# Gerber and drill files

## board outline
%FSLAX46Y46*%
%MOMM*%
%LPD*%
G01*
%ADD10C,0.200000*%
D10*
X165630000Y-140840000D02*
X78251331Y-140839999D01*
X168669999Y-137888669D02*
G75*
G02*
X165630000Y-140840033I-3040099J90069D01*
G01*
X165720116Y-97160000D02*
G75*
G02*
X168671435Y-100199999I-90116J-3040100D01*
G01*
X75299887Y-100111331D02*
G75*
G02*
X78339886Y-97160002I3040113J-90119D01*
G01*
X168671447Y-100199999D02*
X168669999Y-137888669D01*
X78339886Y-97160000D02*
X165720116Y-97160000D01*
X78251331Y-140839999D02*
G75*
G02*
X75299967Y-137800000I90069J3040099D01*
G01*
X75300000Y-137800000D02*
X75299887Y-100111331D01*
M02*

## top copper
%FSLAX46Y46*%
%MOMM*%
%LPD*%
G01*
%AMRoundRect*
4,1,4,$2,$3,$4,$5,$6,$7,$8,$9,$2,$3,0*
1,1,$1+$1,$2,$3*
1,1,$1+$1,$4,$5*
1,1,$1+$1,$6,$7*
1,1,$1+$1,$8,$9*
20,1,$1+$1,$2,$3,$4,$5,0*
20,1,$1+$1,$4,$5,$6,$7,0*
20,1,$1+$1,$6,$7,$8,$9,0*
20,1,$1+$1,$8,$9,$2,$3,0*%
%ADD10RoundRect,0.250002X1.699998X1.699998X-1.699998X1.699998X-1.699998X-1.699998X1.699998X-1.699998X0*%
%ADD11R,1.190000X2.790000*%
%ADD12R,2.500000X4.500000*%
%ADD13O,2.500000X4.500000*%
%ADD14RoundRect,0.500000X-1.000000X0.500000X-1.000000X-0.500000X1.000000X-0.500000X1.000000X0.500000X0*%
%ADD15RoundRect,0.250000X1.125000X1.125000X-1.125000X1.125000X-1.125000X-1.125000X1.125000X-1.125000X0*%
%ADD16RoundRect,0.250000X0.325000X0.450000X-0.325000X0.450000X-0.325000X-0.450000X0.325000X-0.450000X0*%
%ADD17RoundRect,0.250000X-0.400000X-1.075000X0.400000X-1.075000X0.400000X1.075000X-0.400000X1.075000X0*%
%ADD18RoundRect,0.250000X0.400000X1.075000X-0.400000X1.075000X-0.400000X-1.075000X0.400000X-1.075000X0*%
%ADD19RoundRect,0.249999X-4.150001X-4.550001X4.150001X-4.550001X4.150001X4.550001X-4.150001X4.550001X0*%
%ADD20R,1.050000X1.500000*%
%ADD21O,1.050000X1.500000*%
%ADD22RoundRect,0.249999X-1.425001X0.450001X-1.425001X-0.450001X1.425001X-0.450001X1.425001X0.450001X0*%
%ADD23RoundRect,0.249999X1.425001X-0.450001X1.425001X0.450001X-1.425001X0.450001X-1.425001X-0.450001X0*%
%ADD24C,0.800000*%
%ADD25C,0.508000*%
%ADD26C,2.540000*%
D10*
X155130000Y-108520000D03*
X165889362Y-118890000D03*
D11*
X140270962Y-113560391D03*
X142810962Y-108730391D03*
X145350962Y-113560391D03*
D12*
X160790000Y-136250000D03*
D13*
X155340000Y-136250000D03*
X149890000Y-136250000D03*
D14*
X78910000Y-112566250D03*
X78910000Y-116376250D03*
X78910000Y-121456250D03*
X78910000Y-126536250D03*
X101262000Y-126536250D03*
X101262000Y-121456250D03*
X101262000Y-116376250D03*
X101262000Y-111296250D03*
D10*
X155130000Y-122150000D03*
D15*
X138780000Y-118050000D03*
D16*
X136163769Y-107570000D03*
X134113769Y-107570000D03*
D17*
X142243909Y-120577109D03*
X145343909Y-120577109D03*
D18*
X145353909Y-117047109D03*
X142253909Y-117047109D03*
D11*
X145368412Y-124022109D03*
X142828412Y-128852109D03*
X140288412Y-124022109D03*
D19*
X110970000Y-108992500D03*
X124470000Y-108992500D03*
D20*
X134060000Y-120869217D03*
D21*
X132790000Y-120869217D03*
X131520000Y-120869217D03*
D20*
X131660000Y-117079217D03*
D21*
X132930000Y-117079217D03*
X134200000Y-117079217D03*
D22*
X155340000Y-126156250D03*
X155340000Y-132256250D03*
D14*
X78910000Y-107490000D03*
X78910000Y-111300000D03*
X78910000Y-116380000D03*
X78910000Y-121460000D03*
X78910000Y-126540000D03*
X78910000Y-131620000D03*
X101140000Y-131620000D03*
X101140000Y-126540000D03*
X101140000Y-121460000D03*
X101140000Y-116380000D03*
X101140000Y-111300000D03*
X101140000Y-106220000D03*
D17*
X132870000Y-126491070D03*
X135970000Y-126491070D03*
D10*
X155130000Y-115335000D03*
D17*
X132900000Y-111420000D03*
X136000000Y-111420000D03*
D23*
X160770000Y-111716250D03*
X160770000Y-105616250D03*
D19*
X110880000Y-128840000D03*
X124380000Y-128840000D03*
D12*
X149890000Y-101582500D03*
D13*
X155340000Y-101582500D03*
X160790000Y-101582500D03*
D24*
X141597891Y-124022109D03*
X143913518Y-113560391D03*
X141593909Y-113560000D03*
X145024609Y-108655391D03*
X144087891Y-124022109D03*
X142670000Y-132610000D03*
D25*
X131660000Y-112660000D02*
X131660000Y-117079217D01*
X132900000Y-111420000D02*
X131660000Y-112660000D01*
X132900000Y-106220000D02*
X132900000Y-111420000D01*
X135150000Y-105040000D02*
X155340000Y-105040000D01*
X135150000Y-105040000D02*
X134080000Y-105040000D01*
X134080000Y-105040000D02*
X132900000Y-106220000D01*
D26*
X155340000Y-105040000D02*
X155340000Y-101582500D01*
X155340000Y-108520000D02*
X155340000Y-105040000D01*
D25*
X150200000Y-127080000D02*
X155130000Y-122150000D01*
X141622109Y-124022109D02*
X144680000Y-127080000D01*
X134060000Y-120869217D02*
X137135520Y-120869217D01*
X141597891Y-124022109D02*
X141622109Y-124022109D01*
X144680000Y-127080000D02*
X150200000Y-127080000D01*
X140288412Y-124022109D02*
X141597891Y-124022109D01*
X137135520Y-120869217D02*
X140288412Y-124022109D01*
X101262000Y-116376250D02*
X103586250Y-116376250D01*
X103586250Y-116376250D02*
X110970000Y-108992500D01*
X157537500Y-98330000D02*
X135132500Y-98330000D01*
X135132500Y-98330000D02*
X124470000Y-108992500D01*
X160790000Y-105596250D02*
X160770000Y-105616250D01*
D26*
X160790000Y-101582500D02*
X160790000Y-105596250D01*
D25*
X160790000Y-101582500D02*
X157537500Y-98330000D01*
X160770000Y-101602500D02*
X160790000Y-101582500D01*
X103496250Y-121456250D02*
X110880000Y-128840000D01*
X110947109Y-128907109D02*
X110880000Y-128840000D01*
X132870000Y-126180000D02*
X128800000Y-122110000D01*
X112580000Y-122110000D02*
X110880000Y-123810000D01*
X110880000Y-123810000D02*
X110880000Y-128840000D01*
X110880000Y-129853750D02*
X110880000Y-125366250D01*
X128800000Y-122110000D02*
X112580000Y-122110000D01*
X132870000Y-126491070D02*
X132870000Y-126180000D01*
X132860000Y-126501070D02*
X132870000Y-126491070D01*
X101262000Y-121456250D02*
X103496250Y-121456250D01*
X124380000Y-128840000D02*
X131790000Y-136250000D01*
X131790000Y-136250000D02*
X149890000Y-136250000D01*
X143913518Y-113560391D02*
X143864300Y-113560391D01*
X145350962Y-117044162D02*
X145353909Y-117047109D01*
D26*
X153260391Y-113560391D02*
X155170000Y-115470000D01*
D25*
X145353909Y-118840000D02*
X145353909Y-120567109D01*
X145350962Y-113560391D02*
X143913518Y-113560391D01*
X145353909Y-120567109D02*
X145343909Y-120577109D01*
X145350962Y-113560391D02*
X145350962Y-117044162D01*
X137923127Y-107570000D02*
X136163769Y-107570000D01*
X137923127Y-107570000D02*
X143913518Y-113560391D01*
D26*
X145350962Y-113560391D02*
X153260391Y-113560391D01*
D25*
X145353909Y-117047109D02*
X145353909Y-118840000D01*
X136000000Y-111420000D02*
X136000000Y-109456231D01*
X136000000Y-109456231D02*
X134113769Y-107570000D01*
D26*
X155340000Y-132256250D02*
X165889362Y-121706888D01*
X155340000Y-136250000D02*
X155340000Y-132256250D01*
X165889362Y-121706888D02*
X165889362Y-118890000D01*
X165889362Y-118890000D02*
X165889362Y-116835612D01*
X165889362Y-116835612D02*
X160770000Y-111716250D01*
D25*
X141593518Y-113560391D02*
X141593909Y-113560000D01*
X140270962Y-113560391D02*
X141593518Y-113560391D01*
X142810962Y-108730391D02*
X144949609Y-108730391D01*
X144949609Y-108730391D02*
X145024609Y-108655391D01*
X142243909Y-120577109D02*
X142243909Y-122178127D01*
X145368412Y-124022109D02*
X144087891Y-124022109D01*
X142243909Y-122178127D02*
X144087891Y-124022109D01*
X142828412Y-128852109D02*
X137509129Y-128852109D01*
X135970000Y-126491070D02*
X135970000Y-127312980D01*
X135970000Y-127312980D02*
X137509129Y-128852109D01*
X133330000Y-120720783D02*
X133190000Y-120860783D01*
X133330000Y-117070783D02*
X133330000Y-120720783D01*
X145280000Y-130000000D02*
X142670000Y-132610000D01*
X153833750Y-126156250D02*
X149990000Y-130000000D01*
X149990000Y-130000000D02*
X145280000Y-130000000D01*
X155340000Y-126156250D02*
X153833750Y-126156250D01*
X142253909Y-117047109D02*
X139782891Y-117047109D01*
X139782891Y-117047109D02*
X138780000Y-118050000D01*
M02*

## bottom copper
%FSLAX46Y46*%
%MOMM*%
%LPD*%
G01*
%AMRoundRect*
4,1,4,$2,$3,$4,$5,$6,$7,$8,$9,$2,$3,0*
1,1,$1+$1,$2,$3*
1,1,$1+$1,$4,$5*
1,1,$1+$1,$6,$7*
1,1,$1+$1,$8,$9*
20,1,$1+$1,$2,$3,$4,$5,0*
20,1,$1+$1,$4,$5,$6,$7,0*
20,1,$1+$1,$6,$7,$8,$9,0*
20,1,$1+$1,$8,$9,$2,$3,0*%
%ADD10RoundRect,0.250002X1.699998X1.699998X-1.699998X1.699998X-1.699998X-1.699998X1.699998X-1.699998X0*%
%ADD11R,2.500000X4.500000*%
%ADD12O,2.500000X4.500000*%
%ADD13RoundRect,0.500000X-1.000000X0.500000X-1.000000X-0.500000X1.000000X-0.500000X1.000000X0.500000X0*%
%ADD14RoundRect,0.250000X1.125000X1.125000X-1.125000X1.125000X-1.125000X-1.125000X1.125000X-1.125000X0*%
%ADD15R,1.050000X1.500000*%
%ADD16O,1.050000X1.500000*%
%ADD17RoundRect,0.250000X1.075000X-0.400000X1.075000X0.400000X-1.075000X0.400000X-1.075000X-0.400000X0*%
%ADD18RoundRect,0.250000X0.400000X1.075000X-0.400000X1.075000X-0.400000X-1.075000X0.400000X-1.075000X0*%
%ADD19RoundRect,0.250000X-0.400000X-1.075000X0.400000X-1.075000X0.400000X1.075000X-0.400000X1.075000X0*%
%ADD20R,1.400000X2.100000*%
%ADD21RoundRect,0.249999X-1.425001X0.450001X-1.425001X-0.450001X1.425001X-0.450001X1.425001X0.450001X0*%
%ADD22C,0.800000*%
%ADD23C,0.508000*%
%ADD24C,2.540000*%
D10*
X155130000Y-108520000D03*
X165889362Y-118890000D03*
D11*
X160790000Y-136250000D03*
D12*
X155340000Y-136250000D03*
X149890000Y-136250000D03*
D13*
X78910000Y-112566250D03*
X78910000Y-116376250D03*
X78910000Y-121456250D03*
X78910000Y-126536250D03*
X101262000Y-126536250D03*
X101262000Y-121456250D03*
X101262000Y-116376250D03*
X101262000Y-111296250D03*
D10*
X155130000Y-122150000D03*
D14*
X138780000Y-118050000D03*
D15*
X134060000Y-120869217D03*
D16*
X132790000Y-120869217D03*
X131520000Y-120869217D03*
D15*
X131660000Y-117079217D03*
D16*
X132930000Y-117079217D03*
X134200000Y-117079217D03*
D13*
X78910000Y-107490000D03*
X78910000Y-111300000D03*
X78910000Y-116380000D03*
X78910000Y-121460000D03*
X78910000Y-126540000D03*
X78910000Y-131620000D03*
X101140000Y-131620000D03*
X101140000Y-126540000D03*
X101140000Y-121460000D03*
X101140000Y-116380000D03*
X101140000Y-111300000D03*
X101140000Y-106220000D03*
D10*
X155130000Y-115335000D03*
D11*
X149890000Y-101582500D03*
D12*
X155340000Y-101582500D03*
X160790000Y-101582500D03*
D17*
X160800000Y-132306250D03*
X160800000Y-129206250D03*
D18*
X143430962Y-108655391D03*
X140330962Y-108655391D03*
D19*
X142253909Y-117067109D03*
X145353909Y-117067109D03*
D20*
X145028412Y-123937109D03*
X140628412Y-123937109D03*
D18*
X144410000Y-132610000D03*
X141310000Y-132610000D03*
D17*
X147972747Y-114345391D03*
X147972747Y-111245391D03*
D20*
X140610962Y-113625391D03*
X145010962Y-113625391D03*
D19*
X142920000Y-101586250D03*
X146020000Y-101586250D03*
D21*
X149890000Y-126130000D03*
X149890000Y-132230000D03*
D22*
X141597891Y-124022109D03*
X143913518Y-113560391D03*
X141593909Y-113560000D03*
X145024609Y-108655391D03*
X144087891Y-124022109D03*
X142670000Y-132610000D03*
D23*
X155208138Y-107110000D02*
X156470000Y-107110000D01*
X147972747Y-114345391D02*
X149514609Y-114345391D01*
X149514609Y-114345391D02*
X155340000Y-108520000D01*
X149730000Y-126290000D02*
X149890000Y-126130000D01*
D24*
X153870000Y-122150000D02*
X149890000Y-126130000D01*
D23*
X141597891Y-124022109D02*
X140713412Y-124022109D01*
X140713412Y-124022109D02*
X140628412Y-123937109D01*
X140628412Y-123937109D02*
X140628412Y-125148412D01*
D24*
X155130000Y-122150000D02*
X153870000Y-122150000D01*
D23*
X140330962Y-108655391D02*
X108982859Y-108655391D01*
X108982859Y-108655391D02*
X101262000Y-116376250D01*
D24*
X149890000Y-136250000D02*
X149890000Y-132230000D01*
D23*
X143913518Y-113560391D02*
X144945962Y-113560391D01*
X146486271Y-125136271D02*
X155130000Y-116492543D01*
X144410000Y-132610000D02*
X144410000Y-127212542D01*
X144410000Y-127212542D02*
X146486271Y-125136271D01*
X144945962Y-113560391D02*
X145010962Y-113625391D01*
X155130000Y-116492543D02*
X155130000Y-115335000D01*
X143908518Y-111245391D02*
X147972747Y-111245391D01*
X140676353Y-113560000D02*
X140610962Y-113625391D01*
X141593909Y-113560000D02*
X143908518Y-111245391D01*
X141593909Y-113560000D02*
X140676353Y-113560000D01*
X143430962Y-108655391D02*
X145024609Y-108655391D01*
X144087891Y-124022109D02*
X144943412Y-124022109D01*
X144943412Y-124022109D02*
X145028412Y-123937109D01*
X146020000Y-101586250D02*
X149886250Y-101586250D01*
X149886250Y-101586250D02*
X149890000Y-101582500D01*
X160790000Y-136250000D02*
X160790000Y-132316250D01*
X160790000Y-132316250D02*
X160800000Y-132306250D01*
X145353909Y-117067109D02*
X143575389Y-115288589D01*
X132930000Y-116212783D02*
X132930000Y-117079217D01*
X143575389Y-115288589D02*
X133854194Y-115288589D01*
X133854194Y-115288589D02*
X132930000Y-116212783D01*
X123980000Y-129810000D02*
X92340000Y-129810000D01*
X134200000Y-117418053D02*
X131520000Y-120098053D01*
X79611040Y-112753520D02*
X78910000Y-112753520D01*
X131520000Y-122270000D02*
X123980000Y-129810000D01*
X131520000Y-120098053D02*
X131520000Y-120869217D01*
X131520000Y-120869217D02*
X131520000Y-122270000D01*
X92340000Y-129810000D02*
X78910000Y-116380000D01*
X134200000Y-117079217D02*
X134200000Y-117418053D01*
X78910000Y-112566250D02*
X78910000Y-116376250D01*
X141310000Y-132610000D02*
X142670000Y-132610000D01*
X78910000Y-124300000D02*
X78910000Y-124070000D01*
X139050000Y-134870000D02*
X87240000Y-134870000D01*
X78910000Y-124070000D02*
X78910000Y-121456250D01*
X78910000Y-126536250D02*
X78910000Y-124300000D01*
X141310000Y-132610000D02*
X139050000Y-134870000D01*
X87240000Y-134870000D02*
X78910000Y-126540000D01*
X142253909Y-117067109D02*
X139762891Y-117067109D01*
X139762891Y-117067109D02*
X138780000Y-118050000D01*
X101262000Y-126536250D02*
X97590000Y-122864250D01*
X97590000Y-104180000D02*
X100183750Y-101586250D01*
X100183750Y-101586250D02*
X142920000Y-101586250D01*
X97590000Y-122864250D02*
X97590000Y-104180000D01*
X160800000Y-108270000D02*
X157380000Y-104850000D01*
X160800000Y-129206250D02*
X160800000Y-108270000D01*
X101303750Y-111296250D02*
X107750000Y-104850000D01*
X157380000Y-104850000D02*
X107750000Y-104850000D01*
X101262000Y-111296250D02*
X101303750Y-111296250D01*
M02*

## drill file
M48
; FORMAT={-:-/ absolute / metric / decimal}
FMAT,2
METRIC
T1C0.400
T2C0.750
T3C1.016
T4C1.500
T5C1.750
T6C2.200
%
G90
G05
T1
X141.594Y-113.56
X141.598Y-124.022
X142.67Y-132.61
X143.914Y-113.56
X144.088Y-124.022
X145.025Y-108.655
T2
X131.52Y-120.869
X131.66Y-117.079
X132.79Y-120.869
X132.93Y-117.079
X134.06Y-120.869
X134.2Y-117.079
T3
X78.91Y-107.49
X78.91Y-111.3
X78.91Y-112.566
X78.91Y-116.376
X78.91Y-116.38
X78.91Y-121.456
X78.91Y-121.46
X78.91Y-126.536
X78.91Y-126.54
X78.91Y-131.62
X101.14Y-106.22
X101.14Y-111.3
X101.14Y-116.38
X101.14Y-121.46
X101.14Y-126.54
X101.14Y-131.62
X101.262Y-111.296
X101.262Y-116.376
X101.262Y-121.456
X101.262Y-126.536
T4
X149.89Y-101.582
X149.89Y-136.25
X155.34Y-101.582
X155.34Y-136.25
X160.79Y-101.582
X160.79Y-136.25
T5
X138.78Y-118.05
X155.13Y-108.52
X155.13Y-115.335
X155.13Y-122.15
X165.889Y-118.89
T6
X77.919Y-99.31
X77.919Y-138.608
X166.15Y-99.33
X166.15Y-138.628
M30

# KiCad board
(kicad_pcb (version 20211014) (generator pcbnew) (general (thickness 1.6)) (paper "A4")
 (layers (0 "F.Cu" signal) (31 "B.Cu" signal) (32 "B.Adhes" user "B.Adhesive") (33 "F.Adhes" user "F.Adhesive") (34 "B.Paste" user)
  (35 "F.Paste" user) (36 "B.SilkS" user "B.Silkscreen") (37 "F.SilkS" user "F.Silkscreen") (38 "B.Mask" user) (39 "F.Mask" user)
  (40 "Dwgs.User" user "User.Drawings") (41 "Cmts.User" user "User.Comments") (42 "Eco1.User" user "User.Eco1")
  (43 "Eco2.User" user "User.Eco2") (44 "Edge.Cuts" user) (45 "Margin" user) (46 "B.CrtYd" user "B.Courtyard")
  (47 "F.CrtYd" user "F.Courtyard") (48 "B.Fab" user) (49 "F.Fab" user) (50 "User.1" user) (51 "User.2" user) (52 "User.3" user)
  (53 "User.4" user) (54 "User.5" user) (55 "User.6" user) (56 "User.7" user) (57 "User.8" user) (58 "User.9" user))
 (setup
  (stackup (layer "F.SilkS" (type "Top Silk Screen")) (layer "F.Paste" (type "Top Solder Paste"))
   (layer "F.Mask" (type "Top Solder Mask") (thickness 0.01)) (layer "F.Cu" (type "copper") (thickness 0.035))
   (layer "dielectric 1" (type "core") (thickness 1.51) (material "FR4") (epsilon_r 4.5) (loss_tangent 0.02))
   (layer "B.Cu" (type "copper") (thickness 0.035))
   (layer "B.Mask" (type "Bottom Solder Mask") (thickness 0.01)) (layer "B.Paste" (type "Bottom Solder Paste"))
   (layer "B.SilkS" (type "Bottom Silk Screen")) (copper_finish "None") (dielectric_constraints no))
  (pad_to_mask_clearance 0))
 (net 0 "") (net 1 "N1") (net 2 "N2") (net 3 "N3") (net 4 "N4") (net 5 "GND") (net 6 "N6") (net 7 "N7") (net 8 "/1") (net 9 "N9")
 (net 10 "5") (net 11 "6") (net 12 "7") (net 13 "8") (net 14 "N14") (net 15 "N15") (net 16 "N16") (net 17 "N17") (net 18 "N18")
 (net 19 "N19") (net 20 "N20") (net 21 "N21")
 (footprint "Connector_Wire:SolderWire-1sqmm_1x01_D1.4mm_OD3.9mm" (layer "F.Cu") (at 155.13 108.52 180)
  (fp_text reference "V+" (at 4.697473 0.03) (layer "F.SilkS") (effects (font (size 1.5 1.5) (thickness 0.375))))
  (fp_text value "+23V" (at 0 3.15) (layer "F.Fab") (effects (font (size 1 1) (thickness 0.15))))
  (pad "1" thru_hole roundrect locked (at 0 0 180) (size 3.9 3.9) (drill 1.75) (layers *.Cu *.Mask) (roundrect_rratio 0.064103) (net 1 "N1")))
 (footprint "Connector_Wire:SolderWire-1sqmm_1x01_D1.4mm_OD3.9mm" (layer "F.Cu") (at 165.889362 118.89 180)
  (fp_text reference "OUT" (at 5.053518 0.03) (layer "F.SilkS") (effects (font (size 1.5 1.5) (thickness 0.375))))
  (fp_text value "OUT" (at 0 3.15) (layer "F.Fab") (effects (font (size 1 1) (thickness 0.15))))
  (pad "1" thru_hole roundrect locked (at 0 0 180) (size 3.9 3.9) (drill 1.75) (layers *.Cu *.Mask) (roundrect_rratio 0.064103) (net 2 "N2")))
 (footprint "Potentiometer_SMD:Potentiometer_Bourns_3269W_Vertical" (layer "F.Cu") (at 142.810962 111.145391 180)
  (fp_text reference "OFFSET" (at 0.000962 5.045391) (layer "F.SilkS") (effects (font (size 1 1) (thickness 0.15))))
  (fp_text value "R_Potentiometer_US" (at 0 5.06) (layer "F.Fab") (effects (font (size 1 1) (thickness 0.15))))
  (pad "1" smd rect locked (at 2.54 -2.415 180) (size 1.19 2.79) (layers "F.Cu" "F.Paste" "F.Mask") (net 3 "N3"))
  (pad "2" smd rect locked (at 0 2.415 180) (size 1.19 2.79) (layers "F.Cu" "F.Paste" "F.Mask") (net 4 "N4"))
  (pad "3" smd rect locked (at -2.54 -2.415 180) (size 1.19 2.79) (layers "F.Cu" "F.Paste" "F.Mask") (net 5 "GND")))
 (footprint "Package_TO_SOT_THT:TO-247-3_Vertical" (layer "F.Cu") (at 160.79 136.25 180)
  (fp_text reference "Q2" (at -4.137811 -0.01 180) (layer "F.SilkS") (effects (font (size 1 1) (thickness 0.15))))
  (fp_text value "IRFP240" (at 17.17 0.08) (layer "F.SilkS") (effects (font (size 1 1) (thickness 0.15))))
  (pad "1" thru_hole rect locked (at 0 0 180) (size 2.5 4.5) (drill 1.5) (layers *.Cu *.Mask) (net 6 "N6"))
  (pad "2" thru_hole oval locked (at 5.45 0 180) (size 2.5 4.5) (drill 1.5) (layers *.Cu *.Mask) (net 2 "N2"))
  (pad "3" thru_hole oval locked (at 10.9 0 180) (size 2.5 4.5) (drill 1.5) (layers *.Cu *.Mask) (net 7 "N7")))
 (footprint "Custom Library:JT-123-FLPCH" (layer "F.Cu") (at 90.34 118.91625 -90)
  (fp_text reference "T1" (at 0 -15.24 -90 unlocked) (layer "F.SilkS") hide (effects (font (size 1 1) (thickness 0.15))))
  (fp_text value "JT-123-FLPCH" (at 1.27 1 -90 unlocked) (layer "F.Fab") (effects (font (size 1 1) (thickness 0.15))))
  (pad "1" thru_hole roundrect locked (at -6.35 11.43 270) (size 2 3) (drill 1.016) (layers *.Cu *.Mask) (roundrect_rratio 0.25)
   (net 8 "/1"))
  (pad "2" thru_hole roundrect locked (at -2.54 11.43 270) (size 2 3) (drill 1.016) (layers *.Cu *.Mask) (roundrect_rratio 0.25)
   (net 8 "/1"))
  (pad "3" thru_hole roundrect locked (at 2.54 11.43 270) (size 2 3) (drill 1.016) (layers *.Cu *.Mask) (roundrect_rratio 0.25) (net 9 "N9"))
  (pad "4" thru_hole roundrect locked (at 7.62 11.43 270) (size 2 3) (drill 1.016) (layers *.Cu *.Mask) (roundrect_rratio 0.25) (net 9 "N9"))
  (pad "5" thru_hole roundrect locked (at 7.62 -10.922 270) (size 2 3) (drill 1.016) (layers *.Cu *.Mask) (roundrect_rratio 0.25)
   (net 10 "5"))
  (pad "6" thru_hole roundrect locked (at 2.54 -10.922 270) (size 2 3) (drill 1.016) (layers *.Cu *.Mask) (roundrect_rratio 0.25)
   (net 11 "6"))
  (pad "7" thru_hole roundrect locked (at -2.54 -10.922 270) (size 2 3) (drill 1.016) (layers *.Cu *.Mask) (roundrect_rratio 0.25)
   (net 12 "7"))
  (pad "8" thru_hole roundrect locked (at -7.62 -10.922 270) (size 2 3) (drill 1.016) (layers *.Cu *.Mask) (roundrect_rratio 0.25)
   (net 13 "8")))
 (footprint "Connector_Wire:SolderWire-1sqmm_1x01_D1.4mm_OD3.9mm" (layer "F.Cu") (at 155.13 122.15 180)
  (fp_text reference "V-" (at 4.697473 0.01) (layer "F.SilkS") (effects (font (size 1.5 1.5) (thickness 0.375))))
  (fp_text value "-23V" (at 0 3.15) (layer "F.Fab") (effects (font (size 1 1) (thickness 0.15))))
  (pad "1" thru_hole roundrect locked (at 0 0 180) (size 3.9 3.9) (drill 1.75) (layers *.Cu *.Mask) (roundrect_rratio 0.064103)
   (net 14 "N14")))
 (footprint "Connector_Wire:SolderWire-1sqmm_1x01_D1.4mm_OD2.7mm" (layer "F.Cu") (at 138.78 118.05 180)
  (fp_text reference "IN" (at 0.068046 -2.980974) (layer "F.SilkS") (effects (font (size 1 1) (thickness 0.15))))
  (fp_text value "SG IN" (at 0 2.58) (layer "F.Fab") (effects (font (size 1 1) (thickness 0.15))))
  (pad "1" thru_hole roundrect locked (at 0 0 180) (size 2.75 2.75) (drill 1.75) (layers *.Cu *.Mask) (roundrect_rratio 0.090909)
   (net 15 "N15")))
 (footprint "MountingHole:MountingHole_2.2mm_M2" (layer "F.Cu") (at 166.15 138.627795)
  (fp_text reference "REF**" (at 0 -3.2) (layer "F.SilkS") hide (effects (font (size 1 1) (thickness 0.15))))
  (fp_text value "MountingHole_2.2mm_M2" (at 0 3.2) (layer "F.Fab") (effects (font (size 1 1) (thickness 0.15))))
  (pad "" np_thru_hole circle locked (at 0 0) (size 2.2 2.2) (drill 2.2) (layers *.Cu *.Mask)))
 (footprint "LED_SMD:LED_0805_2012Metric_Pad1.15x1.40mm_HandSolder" (layer "F.Cu") (at 135.138769 107.57 180)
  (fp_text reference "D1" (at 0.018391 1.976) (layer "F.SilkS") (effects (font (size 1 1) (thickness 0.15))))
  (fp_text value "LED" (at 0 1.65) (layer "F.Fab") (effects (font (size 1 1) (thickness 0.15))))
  (pad "1" smd roundrect locked (at -1.025 0 180) (size 1.15 1.4) (layers "F.Cu" "F.Paste" "F.Mask") (roundrect_rratio 0.217391)
   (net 5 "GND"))
  (pad "2" smd roundrect locked (at 1.025 0 180) (size 1.15 1.4) (layers "F.Cu" "F.Paste" "F.Mask") (roundrect_rratio 0.217391)
   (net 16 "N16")))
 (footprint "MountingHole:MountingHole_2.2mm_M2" (layer "F.Cu") (at 77.918758 99.31)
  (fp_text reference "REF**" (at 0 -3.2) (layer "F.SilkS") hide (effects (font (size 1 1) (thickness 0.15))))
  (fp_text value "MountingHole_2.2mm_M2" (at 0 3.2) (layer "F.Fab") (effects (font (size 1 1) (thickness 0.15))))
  (pad "" np_thru_hole circle locked (at 0 0) (size 2.2 2.2) (drill 2.2) (layers *.Cu *.Mask)))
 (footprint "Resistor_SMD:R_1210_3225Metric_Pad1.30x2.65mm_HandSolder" (layer "F.Cu") (at 143.793909 120.577109)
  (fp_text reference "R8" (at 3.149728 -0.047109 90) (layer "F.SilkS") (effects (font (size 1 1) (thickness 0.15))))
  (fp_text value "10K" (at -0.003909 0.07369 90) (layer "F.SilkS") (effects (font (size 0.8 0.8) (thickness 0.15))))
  (pad "1" smd roundrect locked (at -1.55 0) (size 1.3 2.65) (layers "F.Cu" "F.Paste" "F.Mask") (roundrect_rratio 0.192308) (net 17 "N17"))
  (pad "2" smd roundrect locked (at 1.55 0) (size 1.3 2.65) (layers "F.Cu" "F.Paste" "F.Mask") (roundrect_rratio 0.192308) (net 5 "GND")))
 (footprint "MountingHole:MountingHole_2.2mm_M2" (layer "F.Cu") (at 166.15 99.33)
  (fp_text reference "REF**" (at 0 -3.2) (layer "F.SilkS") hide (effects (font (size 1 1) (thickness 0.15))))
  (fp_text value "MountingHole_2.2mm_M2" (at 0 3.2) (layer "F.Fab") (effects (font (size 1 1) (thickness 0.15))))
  (pad "" np_thru_hole circle locked (at 0 0) (size 2.2 2.2) (drill 2.2) (layers *.Cu *.Mask)))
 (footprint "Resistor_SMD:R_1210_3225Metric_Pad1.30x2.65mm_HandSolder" (layer "F.Cu") (at 143.803909 117.047109 180)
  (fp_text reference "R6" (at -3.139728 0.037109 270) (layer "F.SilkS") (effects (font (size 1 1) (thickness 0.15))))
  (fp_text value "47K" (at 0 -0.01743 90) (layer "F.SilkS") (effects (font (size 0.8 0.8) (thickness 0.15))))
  (pad "1" smd roundrect locked (at -1.55 0 180) (size 1.3 2.65) (layers "F.Cu" "F.Paste" "F.Mask") (roundrect_rratio 0.192308)
   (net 5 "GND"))
  (pad "2" smd roundrect locked (at 1.55 0 180) (size 1.3 2.65) (layers "F.Cu" "F.Paste" "F.Mask") (roundrect_rratio 0.192308)
   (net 15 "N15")))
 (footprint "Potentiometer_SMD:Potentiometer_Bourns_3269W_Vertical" (layer "F.Cu") (at 142.828412 126.437109)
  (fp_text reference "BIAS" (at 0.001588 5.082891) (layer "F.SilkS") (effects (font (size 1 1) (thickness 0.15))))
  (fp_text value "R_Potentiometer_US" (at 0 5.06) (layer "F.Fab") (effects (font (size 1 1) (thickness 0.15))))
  (pad "1" smd rect locked (at 2.54 -2.415) (size 1.19 2.79) (layers "F.Cu" "F.Paste" "F.Mask") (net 17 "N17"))
  (pad "2" smd rect locked (at 0 2.415) (size 1.19 2.79) (layers "F.Cu" "F.Paste" "F.Mask") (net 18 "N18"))
  (pad "3" smd rect locked (at -2.54 -2.415) (size 1.19 2.79) (layers "F.Cu" "F.Paste" "F.Mask") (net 14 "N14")))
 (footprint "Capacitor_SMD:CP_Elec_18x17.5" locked (layer "F.Cu") (at 117.72 108.9925)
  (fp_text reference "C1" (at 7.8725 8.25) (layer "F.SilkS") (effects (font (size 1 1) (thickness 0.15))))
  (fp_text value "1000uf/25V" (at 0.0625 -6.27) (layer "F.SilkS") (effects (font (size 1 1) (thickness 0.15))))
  (pad "1" smd roundrect locked (at -6.75 0) (size 8.8 9.6) (layers "F.Cu" "F.Paste" "F.Mask") (roundrect_rratio 0.028409) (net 12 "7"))
  (pad "2" smd roundrect locked (at 6.75 0) (size 8.8 9.6) (layers "F.Cu" "F.Paste" "F.Mask") (roundrect_rratio 0.028409) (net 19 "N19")))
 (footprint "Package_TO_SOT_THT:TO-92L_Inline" (layer "F.Cu") (at 134.06 120.869217 180)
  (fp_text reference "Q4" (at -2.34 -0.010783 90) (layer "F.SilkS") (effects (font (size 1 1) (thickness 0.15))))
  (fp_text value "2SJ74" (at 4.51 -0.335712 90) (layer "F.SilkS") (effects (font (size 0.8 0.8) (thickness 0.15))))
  (pad "1" thru_hole rect locked (at 0 0 180) (size 1.05 1.5) (drill 0.75) (layers *.Cu *.Mask) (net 14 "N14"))
  (pad "2" thru_hole oval locked (at 1.27 0 180) (size 1.05 1.5) (drill 0.75) (layers *.Cu *.Mask) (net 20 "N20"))
  (pad "3" thru_hole oval locked (at 2.54 0 180) (size 1.05 1.5) (drill 0.75) (layers *.Cu *.Mask) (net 8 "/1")))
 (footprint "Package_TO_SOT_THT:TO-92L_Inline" (layer "F.Cu") (at 131.66 117.079217)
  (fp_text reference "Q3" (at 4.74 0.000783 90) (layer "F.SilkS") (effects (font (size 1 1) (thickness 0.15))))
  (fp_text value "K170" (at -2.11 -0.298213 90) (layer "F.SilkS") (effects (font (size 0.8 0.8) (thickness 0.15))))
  (pad "1" thru_hole rect locked (at 0 0) (size 1.05 1.5) (drill 0.75) (layers *.Cu *.Mask) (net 1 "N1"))
  (pad "2" thru_hole oval locked (at 1.27 0) (size 1.05 1.5) (drill 0.75) (layers *.Cu *.Mask) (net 20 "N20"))
  (pad "3" thru_hole oval locked (at 2.54 0) (size 1.05 1.5) (drill 0.75) (layers *.Cu *.Mask) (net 8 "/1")))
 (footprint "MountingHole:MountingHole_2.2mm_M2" (layer "F.Cu") (at 77.918758 138.607795)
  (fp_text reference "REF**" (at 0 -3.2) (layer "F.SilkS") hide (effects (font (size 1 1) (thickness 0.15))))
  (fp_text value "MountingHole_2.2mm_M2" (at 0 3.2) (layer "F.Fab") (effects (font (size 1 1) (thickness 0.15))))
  (pad "" np_thru_hole circle locked (at 0 0) (size 2.2 2.2) (drill 2.2) (layers *.Cu *.Mask)))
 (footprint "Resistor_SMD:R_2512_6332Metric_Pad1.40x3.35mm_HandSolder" (layer "F.Cu") (at 155.34 129.20625 -90)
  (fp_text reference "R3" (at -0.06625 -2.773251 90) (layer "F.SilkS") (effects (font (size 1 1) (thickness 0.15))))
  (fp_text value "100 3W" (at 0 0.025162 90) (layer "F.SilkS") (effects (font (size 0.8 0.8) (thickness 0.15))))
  (pad "1" smd roundrect locked (at -3.05 0 270) (size 1.4 3.35) (layers "F.Cu" "F.Paste" "F.Mask") (roundrect_rratio 0.178571) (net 9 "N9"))
  (pad "2" smd roundrect locked (at 3.05 0 270) (size 1.4 3.35) (layers "F.Cu" "F.Paste" "F.Mask") (roundrect_rratio 0.178571) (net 2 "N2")))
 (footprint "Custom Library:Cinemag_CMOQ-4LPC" (layer "F.Cu") (at 90.025 118.92 -90)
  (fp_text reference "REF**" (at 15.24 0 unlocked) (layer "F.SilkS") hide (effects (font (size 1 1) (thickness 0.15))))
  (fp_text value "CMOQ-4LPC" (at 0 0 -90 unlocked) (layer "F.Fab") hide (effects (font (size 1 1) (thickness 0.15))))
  (pad "1" thru_hole roundrect (at -11.43 11.115 270) (size 2 3) (drill 1.016) (layers *.Cu *.Mask) (roundrect_rratio 0.25))
  (pad "2" thru_hole roundrect (at -7.62 11.115 270) (size 2 3) (drill 1.016) (layers *.Cu *.Mask) (roundrect_rratio 0.25) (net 8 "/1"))
  (pad "3" thru_hole roundrect (at -2.54 11.115 270) (size 2 3) (drill 1.016) (layers *.Cu *.Mask) (roundrect_rratio 0.25) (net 8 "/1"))
  (pad "4" thru_hole roundrect (at 2.54 11.115 270) (size 2 3) (drill 1.016) (layers *.Cu *.Mask) (roundrect_rratio 0.25) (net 9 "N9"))
  (pad "5" thru_hole roundrect (at 7.62 11.115 270) (size 2 3) (drill 1.016) (layers *.Cu *.Mask) (roundrect_rratio 0.25) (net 9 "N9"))
  (pad "6" thru_hole roundrect (at 12.7 11.115 270) (size 2 3) (drill 1.016) (layers *.Cu *.Mask) (roundrect_rratio 0.25))
  (pad "7" thru_hole roundrect (at 12.7 -11.115 270) (size 2 3) (drill 1.016) (layers *.Cu *.Mask) (roundrect_rratio 0.25))
  (pad "8" thru_hole roundrect (at 7.62 -11.115 270) (size 2 3) (drill 1.016) (layers *.Cu *.Mask) (roundrect_rratio 0.25))
  (pad "9" thru_hole roundrect (at 2.54 -11.115 270) (size 2 3) (drill 1.016) (layers *.Cu *.Mask) (roundrect_rratio 0.25))
  (pad "10" thru_hole roundrect (at -2.54 -11.115 270) (size 2 3) (drill 1.016) (layers *.Cu *.Mask) (roundrect_rratio 0.25))
  (pad "11" thru_hole roundrect (at -7.62 -11.115 270) (size 2 3) (drill 1.016) (layers *.Cu *.Mask) (roundrect_rratio 0.25) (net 13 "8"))
  (pad "12" thru_hole roundrect (at -12.7 -11.115 270) (size 2 3) (drill 1.016) (layers *.Cu *.Mask) (roundrect_rratio 0.25)))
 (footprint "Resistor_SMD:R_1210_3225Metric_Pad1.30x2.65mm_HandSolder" (layer "F.Cu") (at 134.42 126.49107)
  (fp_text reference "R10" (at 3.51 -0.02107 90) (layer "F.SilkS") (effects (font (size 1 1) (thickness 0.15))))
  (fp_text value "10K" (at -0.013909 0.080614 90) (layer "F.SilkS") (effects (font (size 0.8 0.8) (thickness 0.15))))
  (pad "1" smd roundrect locked (at -1.55 0) (size 1.3 2.65) (layers "F.Cu" "F.Paste" "F.Mask") (roundrect_rratio 0.192308) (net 11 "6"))
  (pad "2" smd roundrect locked (at 1.55 0) (size 1.3 2.65) (layers "F.Cu" "F.Paste" "F.Mask") (roundrect_rratio 0.192308) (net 18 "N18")))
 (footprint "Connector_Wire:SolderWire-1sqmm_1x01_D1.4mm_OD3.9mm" (layer "F.Cu") (at 155.13 115.335 180)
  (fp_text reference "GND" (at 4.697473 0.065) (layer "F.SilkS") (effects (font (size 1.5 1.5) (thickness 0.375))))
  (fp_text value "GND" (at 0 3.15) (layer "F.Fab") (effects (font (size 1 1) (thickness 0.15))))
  (pad "1" thru_hole roundrect locked (at 0 0 180) (size 3.9 3.9) (drill 1.75) (layers *.Cu *.Mask) (roundrect_rratio 0.064103)
   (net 5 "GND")))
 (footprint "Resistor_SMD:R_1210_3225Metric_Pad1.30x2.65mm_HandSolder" (layer "F.Cu") (at 134.45 111.42)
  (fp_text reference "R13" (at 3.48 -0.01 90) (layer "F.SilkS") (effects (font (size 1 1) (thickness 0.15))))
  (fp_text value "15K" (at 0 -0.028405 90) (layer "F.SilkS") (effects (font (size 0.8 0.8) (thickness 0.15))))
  (pad "1" smd roundrect locked (at -1.55 0) (size 1.3 2.65) (layers "F.Cu" "F.Paste" "F.Mask") (roundrect_rratio 0.192308) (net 1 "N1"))
  (pad "2" smd roundrect locked (at 1.55 0) (size 1.3 2.65) (layers "F.Cu" "F.Paste" "F.Mask") (roundrect_rratio 0.192308) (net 16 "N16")))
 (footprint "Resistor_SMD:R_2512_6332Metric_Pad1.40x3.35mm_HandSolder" (layer "F.Cu") (at 160.77 108.66625 90)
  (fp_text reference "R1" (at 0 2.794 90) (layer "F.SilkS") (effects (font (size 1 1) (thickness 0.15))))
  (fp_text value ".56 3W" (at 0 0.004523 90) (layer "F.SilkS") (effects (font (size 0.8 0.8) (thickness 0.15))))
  (pad "1" smd roundrect locked (at -3.05 0 90) (size 1.4 3.35) (layers "F.Cu" "F.Paste" "F.Mask") (roundrect_rratio 0.178571) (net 2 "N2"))
  (pad "2" smd roundrect locked (at 3.05 0 90) (size 1.4 3.35) (layers "F.Cu" "F.Paste" "F.Mask") (roundrect_rratio 0.178571) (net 19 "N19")))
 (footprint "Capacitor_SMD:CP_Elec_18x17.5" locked (layer "F.Cu") (at 117.63 128.84)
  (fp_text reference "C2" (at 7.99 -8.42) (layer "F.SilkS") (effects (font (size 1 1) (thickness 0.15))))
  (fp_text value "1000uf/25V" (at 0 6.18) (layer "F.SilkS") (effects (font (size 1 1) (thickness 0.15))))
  (pad "1" smd roundrect locked (at -6.75 0) (size 8.8 9.6) (layers "F.Cu" "F.Paste" "F.Mask") (roundrect_rratio 0.028409) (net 11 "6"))
  (pad "2" smd roundrect locked (at 6.75 0) (size 8.8 9.6) (layers "F.Cu" "F.Paste" "F.Mask") (roundrect_rratio 0.028409) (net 7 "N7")))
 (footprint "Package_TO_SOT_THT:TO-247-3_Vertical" (layer "F.Cu") (at 149.89 101.5825)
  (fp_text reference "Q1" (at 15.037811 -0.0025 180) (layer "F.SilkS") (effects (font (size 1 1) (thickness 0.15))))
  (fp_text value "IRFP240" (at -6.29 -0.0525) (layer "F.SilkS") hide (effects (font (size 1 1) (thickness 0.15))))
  (pad "1" thru_hole rect locked (at 0 0) (size 2.5 4.5) (drill 1.5) (layers *.Cu *.Mask) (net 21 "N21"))
  (pad "2" thru_hole oval locked (at 5.45 0) (size 2.5 4.5) (drill 1.5) (layers *.Cu *.Mask) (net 1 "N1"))
  (pad "3" thru_hole oval locked (at 10.9 0) (size 2.5 4.5) (drill 1.5) (layers *.Cu *.Mask) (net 19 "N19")))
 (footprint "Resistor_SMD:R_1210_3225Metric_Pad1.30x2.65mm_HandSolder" (layer "B.Cu") (at 160.8 130.75625 90)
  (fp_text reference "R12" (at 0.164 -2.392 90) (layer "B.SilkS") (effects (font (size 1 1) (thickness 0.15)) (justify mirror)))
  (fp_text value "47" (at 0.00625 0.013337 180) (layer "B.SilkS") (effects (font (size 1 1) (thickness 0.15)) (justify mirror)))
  (pad "1" smd roundrect locked (at -1.55 0 90) (size 1.3 2.65) (layers "B.Cu" "B.Paste" "B.Mask") (roundrect_rratio 0.192308) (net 6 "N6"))
  (pad "2" smd roundrect locked (at 1.55 0 90) (size 1.3 2.65) (layers "B.Cu" "B.Paste" "B.Mask") (roundrect_rratio 0.192308) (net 13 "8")))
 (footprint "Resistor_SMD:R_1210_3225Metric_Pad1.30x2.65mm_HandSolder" (layer "B.Cu") (at 141.880962 108.655391 180)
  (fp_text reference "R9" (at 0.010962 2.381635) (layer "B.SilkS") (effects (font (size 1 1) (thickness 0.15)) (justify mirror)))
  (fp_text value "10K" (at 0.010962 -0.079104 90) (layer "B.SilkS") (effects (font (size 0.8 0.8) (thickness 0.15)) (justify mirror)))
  (pad "1" smd roundrect locked (at -1.55 0 180) (size 1.3 2.65) (layers "B.Cu" "B.Paste" "B.Mask") (roundrect_rratio 0.192308) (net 4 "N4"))
  (pad "2" smd roundrect locked (at 1.55 0 180) (size 1.3 2.65) (layers "B.Cu" "B.Paste" "B.Mask") (roundrect_rratio 0.192308) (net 12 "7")))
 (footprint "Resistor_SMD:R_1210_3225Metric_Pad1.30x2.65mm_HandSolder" (layer "B.Cu") (at 143.803909 117.067109)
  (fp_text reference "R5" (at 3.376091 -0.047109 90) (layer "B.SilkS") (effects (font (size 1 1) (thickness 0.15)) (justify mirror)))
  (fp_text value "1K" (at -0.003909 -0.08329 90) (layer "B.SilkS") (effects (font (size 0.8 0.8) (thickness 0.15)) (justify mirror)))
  (pad "1" smd roundrect locked (at -1.55 0) (size 1.3 2.65) (layers "B.Cu" "B.Paste" "B.Mask") (roundrect_rratio 0.192308) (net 15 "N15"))
  (pad "2" smd roundrect locked (at 1.55 0) (size 1.3 2.65) (layers "B.Cu" "B.Paste" "B.Mask") (roundrect_rratio 0.192308) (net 20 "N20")))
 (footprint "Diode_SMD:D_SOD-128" (layer "B.Cu") (at 142.828412 123.937109 180)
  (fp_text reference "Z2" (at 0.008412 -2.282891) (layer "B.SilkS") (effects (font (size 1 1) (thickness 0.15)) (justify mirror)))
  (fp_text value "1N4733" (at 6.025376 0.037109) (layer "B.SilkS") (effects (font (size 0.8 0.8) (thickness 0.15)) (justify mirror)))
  (pad "1" smd rect locked (at -2.2 0 180) (size 1.4 2.1) (layers "B.Cu" "B.Paste" "B.Mask") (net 17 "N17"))
  (pad "2" smd rect locked (at 2.2 0 180) (size 1.4 2.1) (layers "B.Cu" "B.Paste" "B.Mask") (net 14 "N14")))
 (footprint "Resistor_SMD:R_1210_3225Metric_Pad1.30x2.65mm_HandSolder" (layer "B.Cu") (at 142.86 132.61 180)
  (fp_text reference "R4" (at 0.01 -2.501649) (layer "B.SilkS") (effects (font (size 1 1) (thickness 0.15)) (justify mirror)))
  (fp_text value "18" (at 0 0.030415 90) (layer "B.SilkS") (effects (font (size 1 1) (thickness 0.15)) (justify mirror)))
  (pad "1" smd roundrect locked (at -1.55 0 180) (size 1.3 2.65) (layers "B.Cu" "B.Paste" "B.Mask") (roundrect_rratio 0.192308)
   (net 5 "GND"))
  (pad "2" smd roundrect locked (at 1.55 0 180) (size 1.3 2.65) (layers "B.Cu" "B.Paste" "B.Mask") (roundrect_rratio 0.192308) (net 9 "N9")))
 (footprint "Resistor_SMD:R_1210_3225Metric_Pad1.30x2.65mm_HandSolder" (layer "B.Cu") (at 147.972747 112.795391 90)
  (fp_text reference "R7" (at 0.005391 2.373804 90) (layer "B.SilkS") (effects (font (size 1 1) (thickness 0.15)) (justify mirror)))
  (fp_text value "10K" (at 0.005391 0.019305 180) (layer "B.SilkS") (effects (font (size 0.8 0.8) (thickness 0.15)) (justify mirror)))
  (pad "1" smd roundrect locked (at -1.55 0 90) (size 1.3 2.65) (layers "B.Cu" "B.Paste" "B.Mask") (roundrect_rratio 0.192308) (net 1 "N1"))
  (pad "2" smd roundrect locked (at 1.55 0 90) (size 1.3 2.65) (layers "B.Cu" "B.Paste" "B.Mask") (roundrect_rratio 0.192308) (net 3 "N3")))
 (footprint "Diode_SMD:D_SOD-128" (layer "B.Cu") (at 142.810962 113.625391)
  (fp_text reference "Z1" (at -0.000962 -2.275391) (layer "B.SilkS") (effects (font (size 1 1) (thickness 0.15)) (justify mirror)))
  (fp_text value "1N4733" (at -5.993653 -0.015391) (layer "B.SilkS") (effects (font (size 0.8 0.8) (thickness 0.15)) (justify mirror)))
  (pad "1" smd rect locked (at -2.2 0) (size 1.4 2.1) (layers "B.Cu" "B.Paste" "B.Mask") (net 3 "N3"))
  (pad "2" smd rect locked (at 2.2 0) (size 1.4 2.1) (layers "B.Cu" "B.Paste" "B.Mask") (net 5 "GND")))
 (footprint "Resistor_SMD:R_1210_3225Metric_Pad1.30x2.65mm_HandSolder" (layer "B.Cu") (at 144.47 101.58625)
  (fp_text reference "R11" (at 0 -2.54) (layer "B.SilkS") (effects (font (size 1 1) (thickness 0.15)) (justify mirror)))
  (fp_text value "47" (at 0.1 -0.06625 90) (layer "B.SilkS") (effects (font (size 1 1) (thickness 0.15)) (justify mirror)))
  (pad "1" smd roundrect locked (at -1.55 0) (size 1.3 2.65) (layers "B.Cu" "B.Paste" "B.Mask") (roundrect_rratio 0.192308) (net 10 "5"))
  (pad "2" smd roundrect locked (at 1.55 0) (size 1.3 2.65) (layers "B.Cu" "B.Paste" "B.Mask") (roundrect_rratio 0.192308) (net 21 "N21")))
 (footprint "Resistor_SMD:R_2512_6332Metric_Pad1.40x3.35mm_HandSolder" (layer "B.Cu") (at 149.89 129.18 -90)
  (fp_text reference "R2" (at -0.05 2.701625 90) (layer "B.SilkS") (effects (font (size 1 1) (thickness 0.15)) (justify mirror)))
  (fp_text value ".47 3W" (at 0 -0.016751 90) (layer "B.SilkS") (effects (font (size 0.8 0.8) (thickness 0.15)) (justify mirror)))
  (pad "1" smd roundrect locked (at -3.05 0 270) (size 1.4 3.35) (layers "B.Cu" "B.Paste" "B.Mask") (roundrect_rratio 0.178571)
   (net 14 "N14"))
  (pad "2" smd roundrect locked (at 3.05 0 270) (size 1.4 3.35) (layers "B.Cu" "B.Paste" "B.Mask") (roundrect_rratio 0.178571) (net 7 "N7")))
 (gr_line (start 165.63 140.84) (end 78.251331 140.839999) (layer "Edge.Cuts") (width 0.2))
 (gr_arc (start 168.669999 137.888669) (mid 167.748455 139.980769) (end 165.63 140.84) (layer "Edge.Cuts") (width 0.2))
 (gr_arc (start 165.720116 97.16) (mid 167.812216 98.081544) (end 168.671447 100.199999) (layer "Edge.Cuts") (width 0.2))
 (gr_arc (start 75.299887 100.111331) (mid 76.221431 98.019231) (end 78.339886 97.16) (layer "Edge.Cuts") (width 0.2))
 (gr_line (start 168.671447 100.199999) (end 168.669999 137.888669) (layer "Edge.Cuts") (width 0.2))
 (gr_line (start 78.339886 97.16) (end 165.720116 97.16) (layer "Edge.Cuts") (width 0.2))
 (gr_arc (start 78.251331 140.839999) (mid 76.159231 139.918455) (end 75.3 137.8) (layer "Edge.Cuts") (width 0.2))
 (gr_line (start 75.3 137.8) (end 75.299887 100.111331) (layer "Edge.Cuts") (width 0.2))
 (segment (start 131.66 112.66) (end 131.66 117.079217) (width 0.508) (layer "F.Cu") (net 1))
 (segment (start 132.9 111.42) (end 131.66 112.66) (width 0.508) (layer "F.Cu") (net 1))
 (segment (start 132.9 106.22) (end 132.9 111.42) (width 0.508) (layer "F.Cu") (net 1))
 (segment (start 135.15 105.04) (end 155.34 105.04) (width 0.508) (layer "F.Cu") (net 1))
 (segment (start 135.15 105.04) (end 134.08 105.04) (width 0.508) (layer "F.Cu") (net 1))
 (segment (start 134.08 105.04) (end 132.9 106.22) (width 0.508) (layer "F.Cu") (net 1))
 (segment (start 155.34 105.04) (end 155.34 101.5825) (width 2.54) (layer "F.Cu") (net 1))
 (segment (start 155.34 108.52) (end 155.34 105.04) (width 2.54) (layer "F.Cu") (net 1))
 (segment (start 155.208138 107.11) (end 156.47 107.11) (width 0.508) (layer "B.Cu") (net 1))
 (segment (start 147.972747 114.345391) (end 149.514609 114.345391) (width 0.508) (layer "B.Cu") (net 1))
 (segment (start 149.514609 114.345391) (end 155.34 108.52) (width 0.508) (layer "B.Cu") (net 1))
 (segment (start 150.2 127.08) (end 155.13 122.15) (width 0.508) (layer "F.Cu") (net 14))
 (segment (start 141.622109 124.022109) (end 144.68 127.08) (width 0.508) (layer "F.Cu") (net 14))
 (segment (start 134.06 120.869217) (end 137.13552 120.869217) (width 0.508) (layer "F.Cu") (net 14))
 (segment (start 141.597891 124.022109) (end 141.622109 124.022109) (width 0.508) (layer "F.Cu") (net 14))
 (segment (start 144.68 127.08) (end 150.2 127.08) (width 0.508) (layer "F.Cu") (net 14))
 (segment (start 140.288412 124.022109) (end 141.597891 124.022109) (width 0.508) (layer "F.Cu") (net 14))
 (segment (start 137.13552 120.869217) (end 140.288412 124.022109) (width 0.508) (layer "F.Cu") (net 14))
 (via (at 141.597891 124.022109) (size 0.8) (drill 0.4) (layers "F.Cu" "B.Cu") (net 14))
 (segment (start 149.73 126.29) (end 149.89 126.13) (width 0.508) (layer "B.Cu") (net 14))
 (segment (start 153.87 122.15) (end 149.89 126.13) (width 2.54) (layer "B.Cu") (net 14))
 (segment (start 141.597891 124.022109) (end 140.713412 124.022109) (width 0.508) (layer "B.Cu") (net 14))
 (segment (start 140.713412 124.022109) (end 140.628412 123.937109) (width 0.508) (layer "B.Cu") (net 14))
 (segment (start 140.628412 123.937109) (end 140.628412 125.148412) (width 0.508) (layer "B.Cu") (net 14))
 (segment (start 155.13 122.15) (end 153.87 122.15) (width 2.54) (layer "B.Cu") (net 14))
 (segment (start 101.262 116.37625) (end 103.58625 116.37625) (width 0.508) (layer "F.Cu") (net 12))
 (segment (start 103.58625 116.37625) (end 110.97 108.9925) (width 0.508) (layer "F.Cu") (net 12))
 (segment (start 140.330962 108.655391) (end 108.982859 108.655391) (width 0.508) (layer "B.Cu") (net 12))
 (segment (start 108.982859 108.655391) (end 101.262 116.37625) (width 0.508) (layer "B.Cu") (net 12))
 (segment (start 157.5375 98.33) (end 135.1325 98.33) (width 0.508) (layer "F.Cu") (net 19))
 (segment (start 135.1325 98.33) (end 124.47 108.9925) (width 0.508) (layer "F.Cu") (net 19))
 (segment (start 160.79 105.59625) (end 160.77 105.61625) (width 0.508) (layer "F.Cu") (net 19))
 (segment (start 160.79 101.5825) (end 160.79 105.59625) (width 2.54) (layer "F.Cu") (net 19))
 (segment (start 160.79 101.5825) (end 157.5375 98.33) (width 0.508) (layer "F.Cu") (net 19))
 (segment (start 160.77 101.6025) (end 160.79 101.5825) (width 0.508) (layer "F.Cu") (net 19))
 (segment (start 103.49625 121.45625) (end 110.88 128.84) (width 0.508) (layer "F.Cu") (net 11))
 (segment (start 110.947109 128.907109) (end 110.88 128.84) (width 0.508) (layer "F.Cu") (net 11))
 (segment (start 132.87 126.18) (end 128.8 122.11) (width 0.508) (layer "F.Cu") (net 11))
 (segment (start 112.58 122.11) (end 110.88 123.81) (width 0.508) (layer "F.Cu") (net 11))
 (segment (start 110.88 123.81) (end 110.88 128.84) (width 0.508) (layer "F.Cu") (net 11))
 (segment (start 110.88 129.85375) (end 110.88 125.36625) (width 0.508) (layer "F.Cu") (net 11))
 (segment (start 128.8 122.11) (end 112.58 122.11) (width 0.508) (layer "F.Cu") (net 11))
 (segment (start 132.87 126.49107) (end 132.87 126.18) (width 0.508) (layer "F.Cu") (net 11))
 (segment (start 132.86 126.50107) (end 132.87 126.49107) (width 0.508) (layer "F.Cu") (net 11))
 (segment (start 101.262 121.45625) (end 103.49625 121.45625) (width 0.508) (layer "F.Cu") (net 11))
 (segment (start 124.38 128.84) (end 131.79 136.25) (width 0.508) (layer "F.Cu") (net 7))
 (segment (start 131.79 136.25) (end 149.89 136.25) (width 0.508) (layer "F.Cu") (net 7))
 (segment (start 149.89 136.25) (end 149.89 132.23) (width 2.54) (layer "B.Cu") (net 7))
 (segment (start 143.913518 113.560391) (end 143.8643 113.560391) (width 0.508) (layer "F.Cu") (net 5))
 (segment (start 145.350962 117.044162) (end 145.353909 117.047109) (width 0.508) (layer "F.Cu") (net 5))
 (segment (start 153.260391 113.560391) (end 155.17 115.47) (width 2.54) (layer "F.Cu") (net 5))
 (segment (start 145.353909 118.84) (end 145.353909 120.567109) (width 0.508) (layer "F.Cu") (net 5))
 (segment (start 145.350962 113.560391) (end 143.913518 113.560391) (width 0.508) (layer "F.Cu") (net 5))
 (segment (start 145.353909 120.567109) (end 145.343909 120.577109) (width 0.508) (layer "F.Cu") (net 5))
 (segment (start 145.350962 113.560391) (end 145.350962 117.044162) (width 0.508) (layer "F.Cu") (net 5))
 (segment (start 137.923127 107.57) (end 136.163769 107.57) (width 0.508) (layer "F.Cu") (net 5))
 (segment (start 137.923127 107.57) (end 143.913518 113.560391) (width 0.508) (layer "F.Cu") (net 5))
 (segment (start 145.350962 113.560391) (end 153.260391 113.560391) (width 2.54) (layer "F.Cu") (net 5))
 (segment (start 145.353909 117.047109) (end 145.353909 118.84) (width 0.508) (layer "F.Cu") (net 5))
 (via (at 143.913518 113.560391) (size 0.8) (drill 0.4) (layers "F.Cu" "B.Cu") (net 5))
 (segment (start 143.913518 113.560391) (end 144.945962 113.560391) (width 0.508) (layer "B.Cu") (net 5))
 (segment (start 146.486271 125.136271) (end 155.13 116.492543) (width 0.508) (layer "B.Cu") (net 5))
 (segment (start 144.41 132.61) (end 144.41 127.212542) (width 0.508) (layer "B.Cu") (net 5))
 (segment (start 144.41 127.212542) (end 146.486271 125.136271) (width 0.508) (layer "B.Cu") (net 5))
 (segment (start 144.945962 113.560391) (end 145.010962 113.625391) (width 0.508) (layer "B.Cu") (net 5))
 (segment (start 155.13 116.492543) (end 155.13 115.335) (width 0.508) (layer "B.Cu") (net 5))
 (segment (start 136 111.42) (end 136 109.456231) (width 0.508) (layer "F.Cu") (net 16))
 (segment (start 136 109.456231) (end 134.113769 107.57) (width 0.508) (layer "F.Cu") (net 16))
 (segment (start 155.34 132.25625) (end 165.889362 121.706888) (width 2.54) (layer "F.Cu") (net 2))
 (segment (start 155.34 136.25) (end 155.34 132.25625) (width 2.54) (layer "F.Cu") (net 2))
 (segment (start 165.889362 121.706888) (end 165.889362 118.89) (width 2.54) (layer "F.Cu") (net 2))
 (segment (start 165.889362 118.89) (end 165.889362 116.835612) (width 2.54) (layer "F.Cu") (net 2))
 (segment (start 165.889362 116.835612) (end 160.77 111.71625) (width 2.54) (layer "F.Cu") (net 2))
 (segment (start 141.593518 113.560391) (end 141.593909 113.56) (width 0.508) (layer "F.Cu") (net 3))
 (segment (start 140.270962 113.560391) (end 141.593518 113.560391) (width 0.508) (layer "F.Cu") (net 3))
 (via (at 141.593909 113.56) (size 0.8) (drill 0.4) (layers "F.Cu" "B.Cu") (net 3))
 (segment (start 143.908518 111.245391) (end 147.972747 111.245391) (width 0.508) (layer "B.Cu") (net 3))
 (segment (start 140.676353 113.56) (end 140.610962 113.625391) (width 0.508) (layer "B.Cu") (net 3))
 (segment (start 141.593909 113.56) (end 143.908518 111.245391) (width 0.508) (layer "B.Cu") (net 3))
 (segment (start 141.593909 113.56) (end 140.676353 113.56) (width 0.508) (layer "B.Cu") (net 3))
 (segment (start 142.810962 108.730391) (end 144.949609 108.730391) (width 0.508) (layer "F.Cu") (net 4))
 (segment (start 144.949609 108.730391) (end 145.024609 108.655391) (width 0.508) (layer "F.Cu") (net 4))
 (via (at 145.024609 108.655391) (size 0.8) (drill 0.4) (layers "F.Cu" "B.Cu") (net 4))
 (segment (start 143.430962 108.655391) (end 145.024609 108.655391) (width 0.508) (layer "B.Cu") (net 4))
 (segment (start 142.243909 120.577109) (end 142.243909 122.178127) (width 0.508) (layer "F.Cu") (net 17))
 (segment (start 145.368412 124.022109) (end 144.087891 124.022109) (width 0.508) (layer "F.Cu") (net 17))
 (segment (start 142.243909 122.178127) (end 144.087891 124.022109) (width 0.508) (layer "F.Cu") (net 17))
 (via (at 144.087891 124.022109) (size 0.8) (drill 0.4) (layers "F.Cu" "B.Cu") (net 17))
 (segment (start 144.087891 124.022109) (end 144.943412 124.022109) (width 0.508) (layer "B.Cu") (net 17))
 (segment (start 144.943412 124.022109) (end 145.028412 123.937109) (width 0.508) (layer "B.Cu") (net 17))
 (segment (start 142.828412 128.852109) (end 137.509129 128.852109) (width 0.508) (layer "F.Cu") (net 18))
 (segment (start 135.97 126.49107) (end 135.97 127.31298) (width 0.508) (layer "F.Cu") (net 18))
 (segment (start 135.97 127.31298) (end 137.509129 128.852109) (width 0.508) (layer "F.Cu") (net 18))
 (segment (start 146.02 101.58625) (end 149.88625 101.58625) (width 0.508) (layer "B.Cu") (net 21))
 (segment (start 149.88625 101.58625) (end 149.89 101.5825) (width 0.508) (layer "B.Cu") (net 21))
 (segment (start 160.79 136.25) (end 160.79 132.31625) (width 0.508) (layer "B.Cu") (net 6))
 (segment (start 160.79 132.31625) (end 160.8 132.30625) (width 0.508) (layer "B.Cu") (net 6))
 (segment (start 133.33 120.720783) (end 133.19 120.860783) (width 0.508) (layer "F.Cu") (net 20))
 (segment (start 133.33 117.070783) (end 133.33 120.720783) (width 0.508) (layer "F.Cu") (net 20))
 (segment (start 145.353909 117.067109) (end 143.575389 115.288589) (width 0.508) (layer "B.Cu") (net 20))
 (segment (start 132.93 116.212783) (end 132.93 117.079217) (width 0.508) (layer "B.Cu") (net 20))
 (segment (start 143.575389 115.288589) (end 133.854194 115.288589) (width 0.508) (layer "B.Cu") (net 20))
 (segment (start 133.854194 115.288589) (end 132.93 116.212783) (width 0.508) (layer "B.Cu") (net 20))
 (segment (start 123.98 129.81) (end 92.34 129.81) (width 0.508) (layer "B.Cu") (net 8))
 (segment (start 134.2 117.418053) (end 131.52 120.098053) (width 0.508) (layer "B.Cu") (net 8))
 (segment (start 79.61104 112.75352) (end 78.91 112.75352) (width 0.508) (layer "B.Cu") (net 8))
 (segment (start 131.52 122.27) (end 123.98 129.81) (width 0.508) (layer "B.Cu") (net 8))
 (segment (start 131.52 120.098053) (end 131.52 120.869217) (width 0.508) (layer "B.Cu") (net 8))
 (segment (start 131.52 120.869217) (end 131.52 122.27) (width 0.508) (layer "B.Cu") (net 8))
 (segment (start 92.34 129.81) (end 78.91 116.38) (width 0.508) (layer "B.Cu") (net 8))
 (segment (start 134.2 117.079217) (end 134.2 117.418053) (width 0.508) (layer "B.Cu") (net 8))
 (segment (start 78.91 112.56625) (end 78.91 116.37625) (width 0.508) (layer "B.Cu") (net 8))
 (segment (start 145.28 130) (end 142.67 132.61) (width 0.508) (layer "F.Cu") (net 9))
 (segment (start 153.83375 126.15625) (end 149.99 130) (width 0.508) (layer "F.Cu") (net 9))
 (segment (start 149.99 130) (end 145.28 130) (width 0.508) (layer "F.Cu") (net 9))
 (segment (start 155.34 126.15625) (end 153.83375 126.15625) (width 0.508) (layer "F.Cu") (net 9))
 (via (at 142.67 132.61) (size 0.8) (drill 0.4) (layers "F.Cu" "B.Cu") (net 9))
 (segment (start 141.31 132.61) (end 142.67 132.61) (width 0.508) (layer "B.Cu") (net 9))
 (segment (start 78.91 124.3) (end 78.91 124.07) (width 0.508) (layer "B.Cu") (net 9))
 (segment (start 139.05 134.87) (end 87.24 134.87) (width 0.508) (layer "B.Cu") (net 9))
 (segment (start 78.91 124.07) (end 78.91 121.45625) (width 0.508) (layer "B.Cu") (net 9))
 (segment (start 78.91 126.53625) (end 78.91 124.3) (width 0.508) (layer "B.Cu") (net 9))
 (segment (start 141.31 132.61) (end 139.05 134.87) (width 0.508) (layer "B.Cu") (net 9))
 (segment (start 87.24 134.87) (end 78.91 126.54) (width 0.508) (layer "B.Cu") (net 9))
 (segment (start 142.253909 117.047109) (end 139.782891 117.047109) (width 0.508) (layer "F.Cu") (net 15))
 (segment (start 139.782891 117.047109) (end 138.78 118.05) (width 0.508) (layer "F.Cu") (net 15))
 (segment (start 142.253909 117.067109) (end 139.762891 117.067109) (width 0.508) (layer "B.Cu") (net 15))
 (segment (start 139.762891 117.067109) (end 138.78 118.05) (width 0.508) (layer "B.Cu") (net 15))
 (segment (start 101.262 126.53625) (end 97.59 122.86425) (width 0.508) (layer "B.Cu") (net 10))
 (segment (start 97.59 104.18) (end 100.18375 101.58625) (width 0.508) (layer "B.Cu") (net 10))
 (segment (start 100.18375 101.58625) (end 142.92 101.58625) (width 0.508) (layer "B.Cu") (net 10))
 (segment (start 97.59 122.86425) (end 97.59 104.18) (width 0.508) (layer "B.Cu") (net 10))
 (segment (start 160.8 108.27) (end 157.38 104.85) (width 0.508) (layer "B.Cu") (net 13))
 (segment (start 160.8 129.20625) (end 160.8 108.27) (width 0.508) (layer "B.Cu") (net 13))
 (segment (start 101.30375 111.29625) (end 107.75 104.85) (width 0.508) (layer "B.Cu") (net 13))
 (segment (start 157.38 104.85) (end 107.75 104.85) (width 0.508) (layer "B.Cu") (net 13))
 (segment (start 101.262 111.29625) (end 101.30375 111.29625) (width 0.508) (layer "B.Cu") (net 13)))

